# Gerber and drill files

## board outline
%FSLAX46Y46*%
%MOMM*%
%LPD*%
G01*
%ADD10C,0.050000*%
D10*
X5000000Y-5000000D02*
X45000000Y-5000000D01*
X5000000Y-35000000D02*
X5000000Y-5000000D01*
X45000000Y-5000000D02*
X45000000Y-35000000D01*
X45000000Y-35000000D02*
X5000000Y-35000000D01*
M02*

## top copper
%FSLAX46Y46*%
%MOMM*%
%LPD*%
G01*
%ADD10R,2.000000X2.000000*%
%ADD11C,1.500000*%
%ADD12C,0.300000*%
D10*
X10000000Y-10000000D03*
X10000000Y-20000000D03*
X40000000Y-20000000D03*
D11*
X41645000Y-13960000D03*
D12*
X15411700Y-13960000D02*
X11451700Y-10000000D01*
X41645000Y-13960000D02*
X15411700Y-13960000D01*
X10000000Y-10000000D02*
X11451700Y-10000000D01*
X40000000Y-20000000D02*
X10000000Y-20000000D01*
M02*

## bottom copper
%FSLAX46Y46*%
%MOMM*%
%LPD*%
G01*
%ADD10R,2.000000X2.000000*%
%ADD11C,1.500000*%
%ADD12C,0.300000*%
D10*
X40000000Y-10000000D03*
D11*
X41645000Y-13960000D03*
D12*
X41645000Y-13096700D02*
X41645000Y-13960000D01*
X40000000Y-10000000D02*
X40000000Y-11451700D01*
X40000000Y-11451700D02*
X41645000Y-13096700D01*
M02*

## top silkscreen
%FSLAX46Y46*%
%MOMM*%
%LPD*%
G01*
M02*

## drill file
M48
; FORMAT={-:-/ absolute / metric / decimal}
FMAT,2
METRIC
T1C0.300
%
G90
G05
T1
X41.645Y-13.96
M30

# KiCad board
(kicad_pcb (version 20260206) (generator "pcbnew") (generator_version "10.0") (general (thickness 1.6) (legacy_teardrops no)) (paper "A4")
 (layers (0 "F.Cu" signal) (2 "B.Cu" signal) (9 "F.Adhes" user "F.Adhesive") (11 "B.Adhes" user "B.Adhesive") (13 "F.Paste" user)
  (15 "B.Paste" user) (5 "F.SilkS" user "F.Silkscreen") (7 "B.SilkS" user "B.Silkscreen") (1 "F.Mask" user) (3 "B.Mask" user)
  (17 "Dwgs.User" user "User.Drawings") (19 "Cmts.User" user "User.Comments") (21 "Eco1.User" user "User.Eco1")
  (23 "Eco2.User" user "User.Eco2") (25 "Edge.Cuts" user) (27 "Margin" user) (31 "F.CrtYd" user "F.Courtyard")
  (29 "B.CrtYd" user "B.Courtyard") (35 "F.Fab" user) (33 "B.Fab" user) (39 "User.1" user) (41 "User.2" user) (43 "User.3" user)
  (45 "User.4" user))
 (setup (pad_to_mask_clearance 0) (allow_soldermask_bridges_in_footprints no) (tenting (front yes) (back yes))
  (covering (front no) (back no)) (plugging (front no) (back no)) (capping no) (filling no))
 (gr_line (start 5 5) (end 45 5) (stroke (width 0.05) (type default)) (layer "Edge.Cuts"))
 (gr_line (start 5 35) (end 5 5) (stroke (width 0.05) (type default)) (layer "Edge.Cuts"))
 (gr_line (start 45 5) (end 45 35) (stroke (width 0.05) (type default)) (layer "Edge.Cuts"))
 (gr_line (start 45 35) (end 5 35) (stroke (width 0.05) (type default)) (layer "Edge.Cuts"))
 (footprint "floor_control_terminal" (layer "F.Cu") (at 10 10)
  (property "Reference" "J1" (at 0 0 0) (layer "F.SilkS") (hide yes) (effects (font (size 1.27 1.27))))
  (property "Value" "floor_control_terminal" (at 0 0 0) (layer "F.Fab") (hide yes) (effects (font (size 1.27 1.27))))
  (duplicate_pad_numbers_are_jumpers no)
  (pad "1" smd rect (at 0 0) (size 2 2) (layers "F.Cu" "F.Paste" "F.Mask") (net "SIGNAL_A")))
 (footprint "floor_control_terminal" (layer "B.Cu") (at 40 10)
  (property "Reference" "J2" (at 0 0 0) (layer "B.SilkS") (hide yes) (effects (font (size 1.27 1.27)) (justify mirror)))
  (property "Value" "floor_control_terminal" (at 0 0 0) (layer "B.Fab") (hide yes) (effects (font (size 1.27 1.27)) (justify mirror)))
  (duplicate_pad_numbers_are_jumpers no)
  (pad "1" smd rect (at 0 0) (size 2 2) (layers "B.Cu" "B.Paste" "B.Mask") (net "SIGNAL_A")))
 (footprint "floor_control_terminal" (layer "F.Cu") (at 10 20)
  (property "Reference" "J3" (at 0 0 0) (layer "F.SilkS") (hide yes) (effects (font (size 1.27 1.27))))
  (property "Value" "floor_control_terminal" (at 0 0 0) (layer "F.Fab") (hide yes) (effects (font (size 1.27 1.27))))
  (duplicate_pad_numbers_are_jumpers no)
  (pad "1" smd rect (at 0 0) (size 2 2) (layers "F.Cu" "F.Paste" "F.Mask") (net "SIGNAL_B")))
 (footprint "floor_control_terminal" (layer "F.Cu") (at 40 20)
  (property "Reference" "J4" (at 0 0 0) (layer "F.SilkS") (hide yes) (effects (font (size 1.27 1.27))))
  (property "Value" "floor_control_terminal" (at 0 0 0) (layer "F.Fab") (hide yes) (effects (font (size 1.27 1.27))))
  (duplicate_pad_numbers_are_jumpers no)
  (pad "1" smd rect (at 0 0) (size 2 2) (layers "F.Cu" "F.Paste" "F.Mask") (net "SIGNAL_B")))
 (segment (start 15.4117 13.96) (end 11.4517 10) (width 0.3) (layer "F.Cu") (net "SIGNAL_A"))
 (segment (start 41.645 13.96) (end 15.4117 13.96) (width 0.3) (layer "F.Cu") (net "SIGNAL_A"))
 (segment (start 10 10) (end 11.4517 10) (width 0.3) (layer "F.Cu") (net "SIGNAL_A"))
 (via (at 41.645 13.96) (size 1.5) (drill 0.3) (layers "F.Cu" "B.Cu") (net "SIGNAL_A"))
 (segment (start 41.645 13.0967) (end 41.645 13.96) (width 0.3) (layer "B.Cu") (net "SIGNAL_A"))
 (segment (start 40 10) (end 40 11.4517) (width 0.3) (layer "B.Cu") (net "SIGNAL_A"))
 (segment (start 40 11.4517) (end 41.645 13.0967) (width 0.3) (layer "B.Cu") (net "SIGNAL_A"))
 (segment (start 40 20) (end 10 20) (width 0.3) (layer "F.Cu") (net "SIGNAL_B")))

